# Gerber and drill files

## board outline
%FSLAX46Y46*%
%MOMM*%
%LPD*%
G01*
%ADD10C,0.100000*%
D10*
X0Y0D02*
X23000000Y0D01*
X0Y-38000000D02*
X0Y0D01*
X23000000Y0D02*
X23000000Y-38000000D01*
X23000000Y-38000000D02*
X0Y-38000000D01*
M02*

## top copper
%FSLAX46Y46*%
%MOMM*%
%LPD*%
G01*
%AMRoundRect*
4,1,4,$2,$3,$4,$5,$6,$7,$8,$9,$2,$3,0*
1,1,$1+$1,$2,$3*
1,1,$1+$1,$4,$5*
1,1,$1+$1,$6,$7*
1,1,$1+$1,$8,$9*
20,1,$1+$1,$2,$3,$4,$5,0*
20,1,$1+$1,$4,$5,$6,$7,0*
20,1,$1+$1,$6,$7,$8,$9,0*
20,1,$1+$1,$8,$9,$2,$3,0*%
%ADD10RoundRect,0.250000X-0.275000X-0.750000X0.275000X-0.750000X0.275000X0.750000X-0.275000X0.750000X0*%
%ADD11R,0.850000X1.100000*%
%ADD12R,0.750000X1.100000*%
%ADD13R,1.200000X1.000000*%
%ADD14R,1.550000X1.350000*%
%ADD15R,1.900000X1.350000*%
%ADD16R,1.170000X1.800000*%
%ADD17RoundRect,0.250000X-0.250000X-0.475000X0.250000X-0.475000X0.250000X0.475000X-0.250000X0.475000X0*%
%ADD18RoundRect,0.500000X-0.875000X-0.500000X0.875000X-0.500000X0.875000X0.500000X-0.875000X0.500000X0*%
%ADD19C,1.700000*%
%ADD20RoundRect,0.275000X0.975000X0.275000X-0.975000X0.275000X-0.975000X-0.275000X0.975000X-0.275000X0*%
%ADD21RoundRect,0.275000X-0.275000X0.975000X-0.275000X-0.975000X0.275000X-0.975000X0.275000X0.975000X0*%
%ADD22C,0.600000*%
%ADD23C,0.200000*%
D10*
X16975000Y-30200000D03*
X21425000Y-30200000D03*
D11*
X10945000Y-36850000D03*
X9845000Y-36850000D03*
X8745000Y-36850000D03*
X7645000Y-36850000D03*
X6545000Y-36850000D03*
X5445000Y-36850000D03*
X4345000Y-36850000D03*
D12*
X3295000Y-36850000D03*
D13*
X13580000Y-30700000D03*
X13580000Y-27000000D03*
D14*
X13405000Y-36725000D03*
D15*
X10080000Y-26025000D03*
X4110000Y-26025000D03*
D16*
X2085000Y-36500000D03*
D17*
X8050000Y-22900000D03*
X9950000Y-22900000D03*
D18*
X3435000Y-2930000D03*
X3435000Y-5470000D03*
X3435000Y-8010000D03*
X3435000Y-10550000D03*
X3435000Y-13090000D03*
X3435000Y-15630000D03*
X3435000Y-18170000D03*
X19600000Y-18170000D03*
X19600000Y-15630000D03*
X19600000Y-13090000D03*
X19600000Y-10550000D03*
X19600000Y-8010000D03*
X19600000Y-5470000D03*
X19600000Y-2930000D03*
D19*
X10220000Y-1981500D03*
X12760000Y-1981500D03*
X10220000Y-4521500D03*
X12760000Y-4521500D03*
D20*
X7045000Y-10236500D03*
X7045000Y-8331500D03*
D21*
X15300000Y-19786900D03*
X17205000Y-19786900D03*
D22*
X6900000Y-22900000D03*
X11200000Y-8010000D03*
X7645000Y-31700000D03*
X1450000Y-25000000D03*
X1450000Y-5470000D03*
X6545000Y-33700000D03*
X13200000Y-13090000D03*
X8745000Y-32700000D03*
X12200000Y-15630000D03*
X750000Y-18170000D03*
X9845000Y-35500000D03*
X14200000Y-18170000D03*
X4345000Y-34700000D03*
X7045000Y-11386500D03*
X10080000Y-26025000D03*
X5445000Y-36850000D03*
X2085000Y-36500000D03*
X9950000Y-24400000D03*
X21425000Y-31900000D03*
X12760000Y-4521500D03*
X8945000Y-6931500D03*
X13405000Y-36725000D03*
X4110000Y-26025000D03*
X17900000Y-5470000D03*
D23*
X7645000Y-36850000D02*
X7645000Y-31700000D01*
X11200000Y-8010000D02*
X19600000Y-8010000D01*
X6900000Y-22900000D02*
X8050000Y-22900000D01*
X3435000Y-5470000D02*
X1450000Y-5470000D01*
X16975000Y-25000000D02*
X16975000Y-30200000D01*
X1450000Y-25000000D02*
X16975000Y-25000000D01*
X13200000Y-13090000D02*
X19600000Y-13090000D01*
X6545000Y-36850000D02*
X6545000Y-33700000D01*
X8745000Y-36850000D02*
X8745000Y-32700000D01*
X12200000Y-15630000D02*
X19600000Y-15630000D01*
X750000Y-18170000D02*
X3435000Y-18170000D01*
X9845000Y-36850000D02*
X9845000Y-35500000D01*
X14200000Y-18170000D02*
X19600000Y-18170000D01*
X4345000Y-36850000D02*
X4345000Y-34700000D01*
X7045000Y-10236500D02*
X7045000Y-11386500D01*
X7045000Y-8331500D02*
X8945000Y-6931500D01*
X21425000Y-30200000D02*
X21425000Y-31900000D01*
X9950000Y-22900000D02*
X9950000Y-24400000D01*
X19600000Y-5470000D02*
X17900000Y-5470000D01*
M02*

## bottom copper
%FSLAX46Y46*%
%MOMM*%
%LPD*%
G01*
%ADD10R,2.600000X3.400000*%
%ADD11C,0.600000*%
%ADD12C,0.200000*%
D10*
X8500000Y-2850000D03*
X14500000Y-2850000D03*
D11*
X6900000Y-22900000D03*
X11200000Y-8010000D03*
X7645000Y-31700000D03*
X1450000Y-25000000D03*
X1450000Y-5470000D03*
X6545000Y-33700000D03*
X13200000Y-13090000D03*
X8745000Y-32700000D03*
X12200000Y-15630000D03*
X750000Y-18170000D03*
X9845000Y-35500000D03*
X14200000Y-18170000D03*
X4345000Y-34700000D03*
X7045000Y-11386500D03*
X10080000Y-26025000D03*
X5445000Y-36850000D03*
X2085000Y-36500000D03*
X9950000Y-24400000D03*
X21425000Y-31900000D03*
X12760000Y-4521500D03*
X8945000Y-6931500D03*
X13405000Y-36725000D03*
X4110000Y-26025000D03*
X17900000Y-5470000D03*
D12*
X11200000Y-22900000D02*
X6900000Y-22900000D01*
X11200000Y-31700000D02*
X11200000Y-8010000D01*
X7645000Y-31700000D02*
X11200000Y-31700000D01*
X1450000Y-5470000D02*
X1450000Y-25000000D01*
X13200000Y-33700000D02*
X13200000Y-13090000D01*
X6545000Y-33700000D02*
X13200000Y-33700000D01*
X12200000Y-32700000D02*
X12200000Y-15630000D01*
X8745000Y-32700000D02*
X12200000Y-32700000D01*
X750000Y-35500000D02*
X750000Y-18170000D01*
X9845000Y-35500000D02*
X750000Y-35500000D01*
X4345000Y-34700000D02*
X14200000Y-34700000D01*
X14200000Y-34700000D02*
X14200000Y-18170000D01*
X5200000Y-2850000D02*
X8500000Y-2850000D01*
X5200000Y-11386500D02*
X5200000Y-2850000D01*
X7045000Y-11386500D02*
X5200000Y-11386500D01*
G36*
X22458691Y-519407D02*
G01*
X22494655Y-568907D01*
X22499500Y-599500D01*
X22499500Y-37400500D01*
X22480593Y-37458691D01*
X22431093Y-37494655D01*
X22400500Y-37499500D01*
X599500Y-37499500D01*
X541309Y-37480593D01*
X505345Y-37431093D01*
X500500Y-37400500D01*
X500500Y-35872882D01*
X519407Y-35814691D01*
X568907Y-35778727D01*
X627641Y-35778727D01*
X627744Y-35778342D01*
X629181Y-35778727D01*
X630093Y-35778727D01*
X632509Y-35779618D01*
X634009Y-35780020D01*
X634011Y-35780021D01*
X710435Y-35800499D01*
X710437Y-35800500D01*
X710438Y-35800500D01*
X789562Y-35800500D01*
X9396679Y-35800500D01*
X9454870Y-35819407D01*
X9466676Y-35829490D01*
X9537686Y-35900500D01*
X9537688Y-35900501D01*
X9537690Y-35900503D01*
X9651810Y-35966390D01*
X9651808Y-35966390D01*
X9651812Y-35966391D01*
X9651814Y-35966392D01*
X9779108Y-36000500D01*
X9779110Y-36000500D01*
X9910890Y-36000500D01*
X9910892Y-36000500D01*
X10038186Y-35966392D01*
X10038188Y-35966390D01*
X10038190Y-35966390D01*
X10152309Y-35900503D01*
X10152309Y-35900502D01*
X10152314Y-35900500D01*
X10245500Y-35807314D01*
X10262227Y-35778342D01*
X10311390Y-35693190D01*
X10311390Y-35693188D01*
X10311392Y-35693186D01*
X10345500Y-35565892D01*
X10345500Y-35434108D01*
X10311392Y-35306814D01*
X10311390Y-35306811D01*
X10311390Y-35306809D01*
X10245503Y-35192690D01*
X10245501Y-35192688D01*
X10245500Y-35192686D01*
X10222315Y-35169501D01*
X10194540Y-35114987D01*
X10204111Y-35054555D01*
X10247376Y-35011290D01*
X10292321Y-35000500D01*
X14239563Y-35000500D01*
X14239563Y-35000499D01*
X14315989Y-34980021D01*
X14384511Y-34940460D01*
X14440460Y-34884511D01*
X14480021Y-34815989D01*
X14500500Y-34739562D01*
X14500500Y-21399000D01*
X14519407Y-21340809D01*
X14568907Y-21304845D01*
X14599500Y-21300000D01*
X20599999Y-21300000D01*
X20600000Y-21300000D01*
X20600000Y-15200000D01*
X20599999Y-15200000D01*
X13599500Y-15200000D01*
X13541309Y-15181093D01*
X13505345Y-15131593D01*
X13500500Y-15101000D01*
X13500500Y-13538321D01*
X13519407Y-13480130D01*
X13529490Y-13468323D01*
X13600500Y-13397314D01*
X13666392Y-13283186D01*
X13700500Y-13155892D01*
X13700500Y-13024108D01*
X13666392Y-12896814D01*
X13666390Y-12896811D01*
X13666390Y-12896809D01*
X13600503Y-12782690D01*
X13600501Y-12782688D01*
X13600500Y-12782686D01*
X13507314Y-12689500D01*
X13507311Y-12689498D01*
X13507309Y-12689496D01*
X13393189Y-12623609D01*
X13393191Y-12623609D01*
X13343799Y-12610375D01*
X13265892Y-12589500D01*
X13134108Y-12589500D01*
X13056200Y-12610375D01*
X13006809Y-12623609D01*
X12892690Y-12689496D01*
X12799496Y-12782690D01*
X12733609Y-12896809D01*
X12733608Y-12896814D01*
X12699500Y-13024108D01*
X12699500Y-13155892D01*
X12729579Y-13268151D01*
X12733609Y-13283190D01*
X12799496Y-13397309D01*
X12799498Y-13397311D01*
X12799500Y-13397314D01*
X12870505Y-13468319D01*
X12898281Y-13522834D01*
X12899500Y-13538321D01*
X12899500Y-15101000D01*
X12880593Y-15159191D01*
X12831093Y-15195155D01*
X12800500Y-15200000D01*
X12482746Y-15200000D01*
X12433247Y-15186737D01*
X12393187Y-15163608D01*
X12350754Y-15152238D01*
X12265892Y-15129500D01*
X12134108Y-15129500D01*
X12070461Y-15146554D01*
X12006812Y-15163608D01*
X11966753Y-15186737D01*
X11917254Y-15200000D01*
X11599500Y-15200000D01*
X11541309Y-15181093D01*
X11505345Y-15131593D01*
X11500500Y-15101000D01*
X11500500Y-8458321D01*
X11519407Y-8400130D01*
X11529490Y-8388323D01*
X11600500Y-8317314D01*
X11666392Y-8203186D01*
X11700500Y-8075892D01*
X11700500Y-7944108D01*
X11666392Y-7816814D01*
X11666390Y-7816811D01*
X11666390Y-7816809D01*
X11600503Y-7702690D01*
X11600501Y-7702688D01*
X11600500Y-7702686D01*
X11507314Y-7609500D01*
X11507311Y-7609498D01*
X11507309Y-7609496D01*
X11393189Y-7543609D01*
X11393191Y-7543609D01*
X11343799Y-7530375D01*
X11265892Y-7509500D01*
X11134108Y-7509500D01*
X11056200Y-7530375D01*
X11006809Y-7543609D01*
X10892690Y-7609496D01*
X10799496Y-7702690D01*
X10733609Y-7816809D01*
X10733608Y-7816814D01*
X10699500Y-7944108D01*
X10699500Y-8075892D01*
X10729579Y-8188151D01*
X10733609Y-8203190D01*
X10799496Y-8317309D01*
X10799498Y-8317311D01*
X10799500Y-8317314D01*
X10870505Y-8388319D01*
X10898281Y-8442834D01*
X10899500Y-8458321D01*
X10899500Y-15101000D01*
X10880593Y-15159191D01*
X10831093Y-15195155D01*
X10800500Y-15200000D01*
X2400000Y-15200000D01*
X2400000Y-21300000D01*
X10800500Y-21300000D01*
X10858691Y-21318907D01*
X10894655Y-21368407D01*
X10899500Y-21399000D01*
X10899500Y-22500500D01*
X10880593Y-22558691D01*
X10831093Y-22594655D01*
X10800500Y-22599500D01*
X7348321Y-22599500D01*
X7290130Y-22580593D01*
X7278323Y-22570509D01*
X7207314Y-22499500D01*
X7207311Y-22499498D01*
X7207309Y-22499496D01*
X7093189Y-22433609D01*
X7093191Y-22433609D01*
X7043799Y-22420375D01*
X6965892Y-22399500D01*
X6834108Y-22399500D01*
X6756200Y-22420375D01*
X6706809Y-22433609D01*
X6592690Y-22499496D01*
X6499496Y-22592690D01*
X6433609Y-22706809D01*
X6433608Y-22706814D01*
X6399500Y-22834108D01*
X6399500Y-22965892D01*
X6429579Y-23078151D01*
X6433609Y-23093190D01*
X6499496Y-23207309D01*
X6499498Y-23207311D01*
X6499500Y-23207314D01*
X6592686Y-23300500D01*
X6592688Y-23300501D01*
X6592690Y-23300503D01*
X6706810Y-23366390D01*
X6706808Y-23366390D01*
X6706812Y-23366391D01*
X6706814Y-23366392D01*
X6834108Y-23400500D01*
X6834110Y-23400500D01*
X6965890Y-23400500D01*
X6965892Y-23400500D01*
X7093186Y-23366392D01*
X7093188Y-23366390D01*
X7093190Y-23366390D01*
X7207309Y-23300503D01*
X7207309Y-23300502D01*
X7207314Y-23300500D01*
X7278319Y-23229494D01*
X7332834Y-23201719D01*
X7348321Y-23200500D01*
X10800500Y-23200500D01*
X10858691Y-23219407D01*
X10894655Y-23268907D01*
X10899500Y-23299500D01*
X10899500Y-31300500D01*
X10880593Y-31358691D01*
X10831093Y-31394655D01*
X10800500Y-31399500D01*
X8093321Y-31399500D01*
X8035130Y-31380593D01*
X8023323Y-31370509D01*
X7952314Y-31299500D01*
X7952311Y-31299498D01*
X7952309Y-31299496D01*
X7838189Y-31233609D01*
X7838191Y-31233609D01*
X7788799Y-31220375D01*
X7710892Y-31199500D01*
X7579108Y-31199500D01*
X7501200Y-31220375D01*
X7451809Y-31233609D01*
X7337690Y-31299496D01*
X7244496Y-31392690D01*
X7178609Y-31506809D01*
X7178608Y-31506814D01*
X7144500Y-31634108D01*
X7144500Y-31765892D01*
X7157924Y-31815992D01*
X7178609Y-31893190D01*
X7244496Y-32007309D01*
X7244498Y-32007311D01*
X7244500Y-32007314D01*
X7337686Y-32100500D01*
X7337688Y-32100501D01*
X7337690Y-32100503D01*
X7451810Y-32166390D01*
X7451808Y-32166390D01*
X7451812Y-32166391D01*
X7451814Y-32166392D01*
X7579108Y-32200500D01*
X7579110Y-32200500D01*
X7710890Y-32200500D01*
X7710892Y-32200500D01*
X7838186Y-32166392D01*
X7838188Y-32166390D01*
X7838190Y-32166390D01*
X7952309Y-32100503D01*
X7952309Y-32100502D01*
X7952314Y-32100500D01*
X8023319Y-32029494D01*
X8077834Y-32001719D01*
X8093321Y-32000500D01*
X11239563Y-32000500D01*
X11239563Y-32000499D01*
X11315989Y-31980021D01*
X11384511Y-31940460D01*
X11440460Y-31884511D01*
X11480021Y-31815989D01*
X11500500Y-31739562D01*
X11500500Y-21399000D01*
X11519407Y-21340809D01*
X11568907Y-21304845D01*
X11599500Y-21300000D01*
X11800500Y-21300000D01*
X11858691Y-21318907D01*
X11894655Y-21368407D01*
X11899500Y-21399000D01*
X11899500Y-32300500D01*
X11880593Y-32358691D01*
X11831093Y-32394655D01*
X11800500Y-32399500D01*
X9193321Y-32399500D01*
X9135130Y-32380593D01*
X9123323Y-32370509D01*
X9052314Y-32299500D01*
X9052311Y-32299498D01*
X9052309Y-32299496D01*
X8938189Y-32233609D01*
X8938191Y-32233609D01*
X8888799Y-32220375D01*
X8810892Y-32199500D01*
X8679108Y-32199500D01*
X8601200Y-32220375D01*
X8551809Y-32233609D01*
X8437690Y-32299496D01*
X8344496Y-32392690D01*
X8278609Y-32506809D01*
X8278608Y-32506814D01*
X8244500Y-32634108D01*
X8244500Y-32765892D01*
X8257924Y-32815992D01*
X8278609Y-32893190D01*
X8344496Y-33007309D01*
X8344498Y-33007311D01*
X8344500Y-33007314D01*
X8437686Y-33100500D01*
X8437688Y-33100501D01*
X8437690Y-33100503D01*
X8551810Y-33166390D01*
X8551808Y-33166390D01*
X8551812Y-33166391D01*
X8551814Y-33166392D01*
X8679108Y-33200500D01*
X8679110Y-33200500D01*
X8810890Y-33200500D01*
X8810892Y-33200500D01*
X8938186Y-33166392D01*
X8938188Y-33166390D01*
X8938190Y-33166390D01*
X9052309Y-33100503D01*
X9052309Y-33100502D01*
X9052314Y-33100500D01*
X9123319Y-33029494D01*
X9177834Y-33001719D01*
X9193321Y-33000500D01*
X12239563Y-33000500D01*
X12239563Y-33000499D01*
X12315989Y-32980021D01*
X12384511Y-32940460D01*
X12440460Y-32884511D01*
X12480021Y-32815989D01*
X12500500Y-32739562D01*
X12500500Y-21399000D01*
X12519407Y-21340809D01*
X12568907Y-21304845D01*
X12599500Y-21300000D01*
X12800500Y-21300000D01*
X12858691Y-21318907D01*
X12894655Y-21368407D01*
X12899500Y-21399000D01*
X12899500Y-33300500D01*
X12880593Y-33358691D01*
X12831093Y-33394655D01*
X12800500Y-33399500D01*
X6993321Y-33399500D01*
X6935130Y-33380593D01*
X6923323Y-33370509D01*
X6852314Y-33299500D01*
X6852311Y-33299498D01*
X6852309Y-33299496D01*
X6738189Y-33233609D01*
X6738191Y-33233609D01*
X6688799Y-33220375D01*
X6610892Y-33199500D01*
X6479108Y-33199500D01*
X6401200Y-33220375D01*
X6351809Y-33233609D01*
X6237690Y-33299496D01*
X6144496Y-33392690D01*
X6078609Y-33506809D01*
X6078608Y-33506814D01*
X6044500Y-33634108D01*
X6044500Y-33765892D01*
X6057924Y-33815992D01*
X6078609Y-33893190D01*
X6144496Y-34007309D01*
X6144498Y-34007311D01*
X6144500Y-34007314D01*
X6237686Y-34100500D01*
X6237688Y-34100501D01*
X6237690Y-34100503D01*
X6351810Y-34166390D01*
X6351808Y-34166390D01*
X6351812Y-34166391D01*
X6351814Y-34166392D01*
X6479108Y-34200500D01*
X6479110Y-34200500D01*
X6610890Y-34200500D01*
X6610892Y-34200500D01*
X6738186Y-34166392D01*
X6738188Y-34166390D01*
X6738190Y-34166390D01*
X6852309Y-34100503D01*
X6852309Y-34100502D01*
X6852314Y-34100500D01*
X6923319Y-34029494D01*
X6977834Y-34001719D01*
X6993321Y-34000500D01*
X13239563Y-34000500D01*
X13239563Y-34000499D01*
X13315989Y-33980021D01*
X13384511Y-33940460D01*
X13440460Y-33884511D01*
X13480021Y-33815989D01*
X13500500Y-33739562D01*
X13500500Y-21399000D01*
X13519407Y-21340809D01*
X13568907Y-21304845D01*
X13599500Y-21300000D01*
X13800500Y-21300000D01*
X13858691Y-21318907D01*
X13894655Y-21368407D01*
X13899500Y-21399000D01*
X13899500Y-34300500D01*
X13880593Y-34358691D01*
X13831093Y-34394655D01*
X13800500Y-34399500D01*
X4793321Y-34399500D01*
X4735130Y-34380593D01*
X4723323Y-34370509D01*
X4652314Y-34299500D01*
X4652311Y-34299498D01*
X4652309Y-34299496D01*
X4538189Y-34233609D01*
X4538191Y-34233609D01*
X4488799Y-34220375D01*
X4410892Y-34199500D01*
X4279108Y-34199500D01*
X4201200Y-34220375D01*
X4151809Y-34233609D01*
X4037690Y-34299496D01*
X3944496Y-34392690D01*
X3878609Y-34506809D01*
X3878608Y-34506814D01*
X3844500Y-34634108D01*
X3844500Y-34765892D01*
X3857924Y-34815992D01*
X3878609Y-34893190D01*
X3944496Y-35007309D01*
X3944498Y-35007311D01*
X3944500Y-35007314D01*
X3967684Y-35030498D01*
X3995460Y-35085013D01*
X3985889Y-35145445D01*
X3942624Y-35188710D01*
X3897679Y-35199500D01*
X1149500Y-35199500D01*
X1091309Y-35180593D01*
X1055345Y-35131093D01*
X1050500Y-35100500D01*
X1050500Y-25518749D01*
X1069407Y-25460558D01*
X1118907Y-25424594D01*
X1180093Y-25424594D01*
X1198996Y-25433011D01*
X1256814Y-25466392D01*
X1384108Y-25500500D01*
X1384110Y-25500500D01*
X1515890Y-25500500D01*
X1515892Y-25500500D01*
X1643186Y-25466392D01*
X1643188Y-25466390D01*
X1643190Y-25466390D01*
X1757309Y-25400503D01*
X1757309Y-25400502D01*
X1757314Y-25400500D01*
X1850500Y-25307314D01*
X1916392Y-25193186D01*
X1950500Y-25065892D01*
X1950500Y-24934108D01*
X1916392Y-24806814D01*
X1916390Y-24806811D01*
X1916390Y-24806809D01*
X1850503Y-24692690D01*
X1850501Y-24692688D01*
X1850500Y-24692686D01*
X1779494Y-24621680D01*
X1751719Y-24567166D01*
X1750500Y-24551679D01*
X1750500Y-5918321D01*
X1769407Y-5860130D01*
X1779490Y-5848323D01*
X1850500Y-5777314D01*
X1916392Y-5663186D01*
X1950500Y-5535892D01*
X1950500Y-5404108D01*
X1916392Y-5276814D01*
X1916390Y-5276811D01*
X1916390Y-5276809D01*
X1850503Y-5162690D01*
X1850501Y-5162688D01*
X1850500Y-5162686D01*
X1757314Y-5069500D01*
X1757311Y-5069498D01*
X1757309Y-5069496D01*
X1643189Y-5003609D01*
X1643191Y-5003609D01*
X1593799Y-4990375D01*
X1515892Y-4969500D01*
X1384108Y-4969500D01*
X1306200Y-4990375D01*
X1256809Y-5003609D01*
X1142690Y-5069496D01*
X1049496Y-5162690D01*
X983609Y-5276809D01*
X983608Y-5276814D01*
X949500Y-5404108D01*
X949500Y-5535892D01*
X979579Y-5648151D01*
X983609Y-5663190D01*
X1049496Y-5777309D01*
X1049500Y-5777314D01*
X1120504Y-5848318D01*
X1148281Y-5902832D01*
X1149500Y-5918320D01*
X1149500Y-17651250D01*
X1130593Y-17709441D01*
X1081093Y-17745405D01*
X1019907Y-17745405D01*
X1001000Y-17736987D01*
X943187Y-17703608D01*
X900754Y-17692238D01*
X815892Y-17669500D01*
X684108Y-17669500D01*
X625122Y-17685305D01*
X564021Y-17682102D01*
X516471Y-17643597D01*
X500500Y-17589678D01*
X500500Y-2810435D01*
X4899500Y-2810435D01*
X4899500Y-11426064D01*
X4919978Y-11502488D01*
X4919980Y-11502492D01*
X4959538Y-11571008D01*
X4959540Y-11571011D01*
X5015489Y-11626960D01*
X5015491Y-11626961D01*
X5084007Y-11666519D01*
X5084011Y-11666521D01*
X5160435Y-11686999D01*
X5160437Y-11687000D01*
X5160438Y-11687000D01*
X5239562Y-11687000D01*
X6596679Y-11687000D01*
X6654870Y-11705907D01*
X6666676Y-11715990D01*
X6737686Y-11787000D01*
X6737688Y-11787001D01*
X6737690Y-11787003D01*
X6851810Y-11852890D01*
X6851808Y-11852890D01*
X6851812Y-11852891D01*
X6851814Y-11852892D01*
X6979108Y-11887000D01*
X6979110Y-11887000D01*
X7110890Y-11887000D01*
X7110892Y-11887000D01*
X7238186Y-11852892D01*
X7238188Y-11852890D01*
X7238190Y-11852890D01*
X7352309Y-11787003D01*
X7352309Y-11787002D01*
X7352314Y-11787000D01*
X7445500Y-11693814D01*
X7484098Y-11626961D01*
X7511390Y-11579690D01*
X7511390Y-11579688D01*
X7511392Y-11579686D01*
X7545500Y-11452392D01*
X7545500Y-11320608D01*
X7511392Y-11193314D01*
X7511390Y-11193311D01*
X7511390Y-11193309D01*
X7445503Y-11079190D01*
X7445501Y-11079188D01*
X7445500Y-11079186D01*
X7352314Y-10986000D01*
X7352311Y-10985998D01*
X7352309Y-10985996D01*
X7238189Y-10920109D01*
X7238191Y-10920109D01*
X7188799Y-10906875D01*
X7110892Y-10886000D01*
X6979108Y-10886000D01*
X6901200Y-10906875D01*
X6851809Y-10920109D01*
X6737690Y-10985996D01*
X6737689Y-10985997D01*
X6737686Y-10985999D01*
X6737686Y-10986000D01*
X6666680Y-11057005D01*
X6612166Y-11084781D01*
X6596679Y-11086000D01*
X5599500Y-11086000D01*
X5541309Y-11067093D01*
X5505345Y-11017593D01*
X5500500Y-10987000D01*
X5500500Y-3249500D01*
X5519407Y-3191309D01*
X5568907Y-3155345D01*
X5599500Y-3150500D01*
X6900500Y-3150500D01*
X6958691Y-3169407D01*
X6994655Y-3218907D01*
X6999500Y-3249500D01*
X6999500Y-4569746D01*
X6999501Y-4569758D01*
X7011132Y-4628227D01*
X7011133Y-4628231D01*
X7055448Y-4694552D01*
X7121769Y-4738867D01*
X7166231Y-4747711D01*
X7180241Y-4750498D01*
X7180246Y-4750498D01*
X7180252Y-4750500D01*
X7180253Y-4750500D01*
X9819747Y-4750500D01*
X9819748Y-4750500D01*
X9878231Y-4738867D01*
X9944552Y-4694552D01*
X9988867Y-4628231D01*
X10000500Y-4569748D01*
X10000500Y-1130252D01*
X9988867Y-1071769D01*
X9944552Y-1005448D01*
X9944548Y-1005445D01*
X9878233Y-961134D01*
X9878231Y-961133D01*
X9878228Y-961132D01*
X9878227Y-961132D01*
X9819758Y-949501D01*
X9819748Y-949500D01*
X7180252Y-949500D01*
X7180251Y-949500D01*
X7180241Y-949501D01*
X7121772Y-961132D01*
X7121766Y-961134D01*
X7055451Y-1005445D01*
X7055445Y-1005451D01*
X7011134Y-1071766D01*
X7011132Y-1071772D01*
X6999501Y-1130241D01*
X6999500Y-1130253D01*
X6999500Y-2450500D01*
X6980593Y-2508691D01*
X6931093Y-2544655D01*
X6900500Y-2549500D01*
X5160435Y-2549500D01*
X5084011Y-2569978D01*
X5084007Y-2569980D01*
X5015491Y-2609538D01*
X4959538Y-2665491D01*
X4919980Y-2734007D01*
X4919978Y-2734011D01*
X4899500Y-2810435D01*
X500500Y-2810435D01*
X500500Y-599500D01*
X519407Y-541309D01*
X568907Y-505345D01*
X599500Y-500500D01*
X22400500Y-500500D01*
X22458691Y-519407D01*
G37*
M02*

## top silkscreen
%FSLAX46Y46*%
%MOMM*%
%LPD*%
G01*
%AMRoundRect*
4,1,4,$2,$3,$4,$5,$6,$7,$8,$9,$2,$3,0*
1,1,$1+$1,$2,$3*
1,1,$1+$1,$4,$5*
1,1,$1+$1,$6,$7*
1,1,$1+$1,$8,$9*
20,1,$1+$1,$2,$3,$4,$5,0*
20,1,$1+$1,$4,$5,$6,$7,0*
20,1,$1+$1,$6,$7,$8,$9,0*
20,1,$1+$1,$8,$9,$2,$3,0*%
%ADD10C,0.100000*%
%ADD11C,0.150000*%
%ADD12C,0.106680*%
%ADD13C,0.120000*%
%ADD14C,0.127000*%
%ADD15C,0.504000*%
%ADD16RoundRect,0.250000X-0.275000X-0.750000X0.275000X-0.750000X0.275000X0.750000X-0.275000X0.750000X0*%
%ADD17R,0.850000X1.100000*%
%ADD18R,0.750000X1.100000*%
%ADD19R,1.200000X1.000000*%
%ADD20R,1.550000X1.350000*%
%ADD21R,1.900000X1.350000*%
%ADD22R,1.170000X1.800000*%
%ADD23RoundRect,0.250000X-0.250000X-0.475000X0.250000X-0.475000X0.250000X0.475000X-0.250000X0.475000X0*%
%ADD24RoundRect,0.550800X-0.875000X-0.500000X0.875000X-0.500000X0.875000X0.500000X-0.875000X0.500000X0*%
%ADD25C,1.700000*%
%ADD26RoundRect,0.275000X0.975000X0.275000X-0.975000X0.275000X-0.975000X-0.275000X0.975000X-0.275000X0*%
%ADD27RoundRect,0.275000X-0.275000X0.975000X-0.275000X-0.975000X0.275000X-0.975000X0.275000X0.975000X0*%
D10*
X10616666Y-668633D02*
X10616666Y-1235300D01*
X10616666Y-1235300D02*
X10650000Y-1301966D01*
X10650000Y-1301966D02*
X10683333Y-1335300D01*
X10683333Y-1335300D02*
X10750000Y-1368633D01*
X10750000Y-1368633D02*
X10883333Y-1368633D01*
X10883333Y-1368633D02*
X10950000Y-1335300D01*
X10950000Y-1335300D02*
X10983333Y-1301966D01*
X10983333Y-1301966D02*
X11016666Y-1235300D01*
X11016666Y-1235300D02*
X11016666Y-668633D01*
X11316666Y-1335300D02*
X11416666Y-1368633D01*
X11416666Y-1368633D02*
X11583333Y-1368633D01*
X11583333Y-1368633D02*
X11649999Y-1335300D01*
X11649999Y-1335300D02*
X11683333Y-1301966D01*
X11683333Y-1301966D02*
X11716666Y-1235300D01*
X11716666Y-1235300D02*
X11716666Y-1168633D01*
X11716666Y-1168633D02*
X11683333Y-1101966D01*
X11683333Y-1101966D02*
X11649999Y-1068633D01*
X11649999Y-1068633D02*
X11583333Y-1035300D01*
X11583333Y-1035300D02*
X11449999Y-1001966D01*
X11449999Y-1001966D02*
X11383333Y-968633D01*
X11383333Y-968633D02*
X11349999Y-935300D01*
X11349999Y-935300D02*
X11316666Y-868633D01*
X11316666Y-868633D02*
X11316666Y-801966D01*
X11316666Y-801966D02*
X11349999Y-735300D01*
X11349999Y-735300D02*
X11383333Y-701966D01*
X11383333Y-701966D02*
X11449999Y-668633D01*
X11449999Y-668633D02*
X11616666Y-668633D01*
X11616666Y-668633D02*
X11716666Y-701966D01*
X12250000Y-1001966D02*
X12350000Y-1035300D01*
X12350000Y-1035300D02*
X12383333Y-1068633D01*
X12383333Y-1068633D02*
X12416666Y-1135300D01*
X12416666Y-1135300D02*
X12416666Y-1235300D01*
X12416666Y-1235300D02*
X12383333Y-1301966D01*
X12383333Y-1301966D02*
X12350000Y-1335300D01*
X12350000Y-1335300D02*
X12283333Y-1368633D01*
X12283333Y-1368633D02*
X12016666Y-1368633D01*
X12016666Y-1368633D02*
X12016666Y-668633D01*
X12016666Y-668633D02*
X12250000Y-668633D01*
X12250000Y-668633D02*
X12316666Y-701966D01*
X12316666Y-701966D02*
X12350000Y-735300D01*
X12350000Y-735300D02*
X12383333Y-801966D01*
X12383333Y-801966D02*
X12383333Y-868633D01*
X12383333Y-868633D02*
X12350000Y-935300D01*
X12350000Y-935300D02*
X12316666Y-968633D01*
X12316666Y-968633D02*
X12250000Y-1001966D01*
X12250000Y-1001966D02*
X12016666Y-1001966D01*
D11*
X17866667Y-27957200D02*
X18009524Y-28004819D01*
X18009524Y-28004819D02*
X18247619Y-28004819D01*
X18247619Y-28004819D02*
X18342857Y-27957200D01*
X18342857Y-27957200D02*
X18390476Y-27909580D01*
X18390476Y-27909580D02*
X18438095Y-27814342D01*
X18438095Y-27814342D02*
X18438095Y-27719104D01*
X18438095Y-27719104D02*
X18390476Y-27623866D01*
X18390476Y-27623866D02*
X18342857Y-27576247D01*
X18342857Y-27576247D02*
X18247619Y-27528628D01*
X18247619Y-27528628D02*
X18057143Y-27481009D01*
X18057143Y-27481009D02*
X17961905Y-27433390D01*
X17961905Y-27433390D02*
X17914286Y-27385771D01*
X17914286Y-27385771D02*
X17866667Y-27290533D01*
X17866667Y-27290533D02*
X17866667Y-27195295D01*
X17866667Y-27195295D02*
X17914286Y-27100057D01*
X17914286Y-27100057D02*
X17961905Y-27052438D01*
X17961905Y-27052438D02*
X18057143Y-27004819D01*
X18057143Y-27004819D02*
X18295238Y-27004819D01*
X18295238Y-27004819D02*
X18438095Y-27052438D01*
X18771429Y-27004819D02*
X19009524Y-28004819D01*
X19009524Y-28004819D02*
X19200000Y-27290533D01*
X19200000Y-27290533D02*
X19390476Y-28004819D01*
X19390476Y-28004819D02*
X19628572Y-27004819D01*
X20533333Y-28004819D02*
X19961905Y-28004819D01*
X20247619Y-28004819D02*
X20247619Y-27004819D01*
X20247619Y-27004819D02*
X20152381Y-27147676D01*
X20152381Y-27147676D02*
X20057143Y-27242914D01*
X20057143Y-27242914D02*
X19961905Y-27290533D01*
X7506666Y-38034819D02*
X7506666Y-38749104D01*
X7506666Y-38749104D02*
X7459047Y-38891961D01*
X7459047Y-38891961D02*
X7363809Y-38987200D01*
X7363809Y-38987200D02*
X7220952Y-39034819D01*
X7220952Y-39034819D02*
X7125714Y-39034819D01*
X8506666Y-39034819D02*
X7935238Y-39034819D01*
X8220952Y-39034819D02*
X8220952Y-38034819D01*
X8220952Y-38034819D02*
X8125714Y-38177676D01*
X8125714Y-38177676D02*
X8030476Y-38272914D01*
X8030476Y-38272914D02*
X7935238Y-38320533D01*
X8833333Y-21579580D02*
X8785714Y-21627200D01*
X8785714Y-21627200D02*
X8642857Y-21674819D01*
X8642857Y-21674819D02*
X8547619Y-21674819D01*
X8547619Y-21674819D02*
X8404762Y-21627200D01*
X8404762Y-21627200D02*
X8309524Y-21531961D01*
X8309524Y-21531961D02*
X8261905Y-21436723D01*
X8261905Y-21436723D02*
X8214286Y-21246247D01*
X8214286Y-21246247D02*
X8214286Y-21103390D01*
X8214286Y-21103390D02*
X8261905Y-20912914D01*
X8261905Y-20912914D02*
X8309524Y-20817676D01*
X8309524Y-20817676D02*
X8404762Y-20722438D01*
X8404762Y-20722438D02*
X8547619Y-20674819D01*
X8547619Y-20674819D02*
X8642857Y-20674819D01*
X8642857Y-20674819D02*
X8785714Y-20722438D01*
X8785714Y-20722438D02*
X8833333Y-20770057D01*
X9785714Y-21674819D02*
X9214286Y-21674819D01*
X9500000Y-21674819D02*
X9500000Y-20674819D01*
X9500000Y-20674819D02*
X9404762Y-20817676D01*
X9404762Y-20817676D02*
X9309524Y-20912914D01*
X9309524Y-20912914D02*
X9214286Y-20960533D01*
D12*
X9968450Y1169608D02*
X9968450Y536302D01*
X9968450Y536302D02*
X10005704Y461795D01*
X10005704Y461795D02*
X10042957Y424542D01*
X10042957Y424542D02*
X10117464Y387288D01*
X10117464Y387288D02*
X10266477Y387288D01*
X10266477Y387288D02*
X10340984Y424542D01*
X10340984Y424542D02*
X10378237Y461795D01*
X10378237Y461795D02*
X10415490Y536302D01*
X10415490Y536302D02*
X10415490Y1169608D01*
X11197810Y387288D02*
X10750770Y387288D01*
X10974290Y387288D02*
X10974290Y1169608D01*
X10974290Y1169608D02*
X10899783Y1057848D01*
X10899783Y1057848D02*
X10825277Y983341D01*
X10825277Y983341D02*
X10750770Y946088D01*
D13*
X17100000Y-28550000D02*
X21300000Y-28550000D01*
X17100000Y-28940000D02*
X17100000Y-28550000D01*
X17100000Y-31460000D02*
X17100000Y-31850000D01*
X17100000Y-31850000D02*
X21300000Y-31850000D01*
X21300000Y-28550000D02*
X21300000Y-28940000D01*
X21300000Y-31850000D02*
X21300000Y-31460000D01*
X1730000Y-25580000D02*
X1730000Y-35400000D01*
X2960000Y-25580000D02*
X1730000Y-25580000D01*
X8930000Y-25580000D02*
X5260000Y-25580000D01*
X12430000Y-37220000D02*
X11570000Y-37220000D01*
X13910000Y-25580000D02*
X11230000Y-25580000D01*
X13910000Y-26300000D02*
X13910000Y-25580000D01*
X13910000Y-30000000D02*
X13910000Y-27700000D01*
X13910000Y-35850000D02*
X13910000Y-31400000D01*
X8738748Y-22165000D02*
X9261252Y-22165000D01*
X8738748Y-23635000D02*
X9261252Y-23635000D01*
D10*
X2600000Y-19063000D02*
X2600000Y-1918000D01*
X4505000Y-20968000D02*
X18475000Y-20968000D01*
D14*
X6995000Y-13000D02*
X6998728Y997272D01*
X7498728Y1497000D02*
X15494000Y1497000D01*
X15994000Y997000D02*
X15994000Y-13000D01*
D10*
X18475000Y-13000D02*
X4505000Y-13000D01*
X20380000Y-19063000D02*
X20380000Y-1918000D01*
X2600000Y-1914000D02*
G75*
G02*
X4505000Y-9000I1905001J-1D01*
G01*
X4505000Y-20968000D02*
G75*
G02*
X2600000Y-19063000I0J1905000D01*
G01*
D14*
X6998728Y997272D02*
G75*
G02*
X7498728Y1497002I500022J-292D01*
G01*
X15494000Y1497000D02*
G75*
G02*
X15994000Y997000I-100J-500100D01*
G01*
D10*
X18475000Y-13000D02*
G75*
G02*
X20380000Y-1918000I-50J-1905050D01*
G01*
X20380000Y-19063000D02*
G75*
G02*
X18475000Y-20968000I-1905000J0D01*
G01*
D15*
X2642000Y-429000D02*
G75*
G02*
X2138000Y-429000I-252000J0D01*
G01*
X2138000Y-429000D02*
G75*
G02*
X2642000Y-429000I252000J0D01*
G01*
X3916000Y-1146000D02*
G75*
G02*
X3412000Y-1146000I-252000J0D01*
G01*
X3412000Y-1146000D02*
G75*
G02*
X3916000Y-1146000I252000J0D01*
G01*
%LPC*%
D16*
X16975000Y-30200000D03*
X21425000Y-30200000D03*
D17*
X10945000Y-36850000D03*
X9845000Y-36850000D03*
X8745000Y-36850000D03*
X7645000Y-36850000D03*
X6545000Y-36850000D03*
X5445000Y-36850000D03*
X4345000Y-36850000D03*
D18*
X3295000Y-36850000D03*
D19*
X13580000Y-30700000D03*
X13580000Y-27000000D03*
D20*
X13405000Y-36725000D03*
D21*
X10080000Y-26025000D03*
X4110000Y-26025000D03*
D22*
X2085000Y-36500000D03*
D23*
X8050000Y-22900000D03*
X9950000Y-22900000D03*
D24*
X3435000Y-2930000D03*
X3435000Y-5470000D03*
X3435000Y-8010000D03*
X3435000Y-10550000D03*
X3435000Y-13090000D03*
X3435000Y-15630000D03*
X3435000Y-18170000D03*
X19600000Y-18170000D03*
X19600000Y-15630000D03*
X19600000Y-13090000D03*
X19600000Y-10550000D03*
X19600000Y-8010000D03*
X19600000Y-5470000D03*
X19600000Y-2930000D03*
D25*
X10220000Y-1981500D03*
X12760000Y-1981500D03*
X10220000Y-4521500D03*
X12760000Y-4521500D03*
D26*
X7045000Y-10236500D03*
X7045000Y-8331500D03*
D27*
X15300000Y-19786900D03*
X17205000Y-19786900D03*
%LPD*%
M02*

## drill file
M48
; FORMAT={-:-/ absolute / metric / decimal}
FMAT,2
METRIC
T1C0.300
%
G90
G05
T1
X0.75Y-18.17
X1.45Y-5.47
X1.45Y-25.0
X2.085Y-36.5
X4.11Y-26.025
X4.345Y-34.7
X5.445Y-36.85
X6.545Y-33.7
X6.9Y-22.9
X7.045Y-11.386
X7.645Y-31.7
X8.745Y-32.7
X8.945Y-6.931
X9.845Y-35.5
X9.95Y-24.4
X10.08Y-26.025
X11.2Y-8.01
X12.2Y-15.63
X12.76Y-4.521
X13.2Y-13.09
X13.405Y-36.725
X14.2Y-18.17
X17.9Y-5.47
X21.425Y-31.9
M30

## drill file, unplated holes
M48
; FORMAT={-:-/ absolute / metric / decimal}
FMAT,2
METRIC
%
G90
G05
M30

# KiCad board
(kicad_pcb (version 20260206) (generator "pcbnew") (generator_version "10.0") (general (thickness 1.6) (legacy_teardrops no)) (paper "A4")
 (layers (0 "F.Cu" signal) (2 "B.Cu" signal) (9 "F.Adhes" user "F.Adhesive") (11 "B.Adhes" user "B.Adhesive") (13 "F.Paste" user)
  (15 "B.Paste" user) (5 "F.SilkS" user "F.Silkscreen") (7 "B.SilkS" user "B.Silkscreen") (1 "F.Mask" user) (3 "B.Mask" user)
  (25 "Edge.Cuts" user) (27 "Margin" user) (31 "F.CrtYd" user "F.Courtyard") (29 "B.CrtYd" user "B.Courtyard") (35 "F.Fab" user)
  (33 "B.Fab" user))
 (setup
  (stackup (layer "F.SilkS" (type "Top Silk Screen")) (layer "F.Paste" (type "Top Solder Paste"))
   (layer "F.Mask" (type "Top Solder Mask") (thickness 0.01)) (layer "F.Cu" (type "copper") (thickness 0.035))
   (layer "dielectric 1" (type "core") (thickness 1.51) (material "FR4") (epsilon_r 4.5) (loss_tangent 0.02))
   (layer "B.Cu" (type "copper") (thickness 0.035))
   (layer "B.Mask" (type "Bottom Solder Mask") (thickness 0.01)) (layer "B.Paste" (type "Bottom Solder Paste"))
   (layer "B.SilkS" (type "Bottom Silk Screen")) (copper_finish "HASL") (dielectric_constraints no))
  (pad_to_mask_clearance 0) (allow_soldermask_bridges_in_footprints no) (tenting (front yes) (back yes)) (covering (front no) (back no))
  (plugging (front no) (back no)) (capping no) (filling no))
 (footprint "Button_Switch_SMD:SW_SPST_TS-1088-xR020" (layer "F.Cu") (at 19.2 30.2)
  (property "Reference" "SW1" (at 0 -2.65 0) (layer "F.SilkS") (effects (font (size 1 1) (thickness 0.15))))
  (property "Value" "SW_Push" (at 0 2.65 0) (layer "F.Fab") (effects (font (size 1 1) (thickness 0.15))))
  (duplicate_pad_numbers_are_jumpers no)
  (fp_line (start -2.1 -1.65) (end 2.1 -1.65) (stroke (width 0.12) (type solid)) (layer "F.SilkS"))
  (fp_line (start -2.1 -1.26) (end -2.1 -1.65) (stroke (width 0.12) (type solid)) (layer "F.SilkS"))
  (fp_line (start -2.1 1.26) (end -2.1 1.65) (stroke (width 0.12) (type solid)) (layer "F.SilkS"))
  (fp_line (start -2.1 1.65) (end 2.1 1.65) (stroke (width 0.12) (type solid)) (layer "F.SilkS"))
  (fp_line (start 2.1 -1.65) (end 2.1 -1.26) (stroke (width 0.12) (type solid)) (layer "F.SilkS"))
  (fp_line (start 2.1 1.65) (end 2.1 1.26) (stroke (width 0.12) (type solid)) (layer "F.SilkS"))
  (pad "1" smd roundrect (at -2.225 0) (size 1.05 2) (layers "F.Cu" "F.Mask" "F.Paste") (roundrect_rratio 0.2380952381) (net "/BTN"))
  (pad "2" smd roundrect (at 2.225 0) (size 1.05 2) (layers "F.Cu" "F.Mask" "F.Paste") (roundrect_rratio 0.2380952381) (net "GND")))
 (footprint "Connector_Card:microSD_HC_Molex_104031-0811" (layer "F.Cu") (at 7.84 31.4 180)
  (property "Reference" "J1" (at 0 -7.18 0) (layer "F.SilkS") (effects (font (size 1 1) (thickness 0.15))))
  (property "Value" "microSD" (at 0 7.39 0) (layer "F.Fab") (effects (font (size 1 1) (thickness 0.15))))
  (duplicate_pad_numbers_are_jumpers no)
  (fp_line (start 6.11 5.82) (end 6.11 -4) (stroke (width 0.12) (type solid)) (layer "F.SilkS"))
  (fp_line (start 4.88 5.82) (end 6.11 5.82) (stroke (width 0.12) (type solid)) (layer "F.SilkS"))
  (fp_line (start -1.09 5.82) (end 2.58 5.82) (stroke (width 0.12) (type solid)) (layer "F.SilkS"))
  (fp_line (start -4.59 -5.82) (end -3.73 -5.82) (stroke (width 0.12) (type solid)) (layer "F.SilkS"))
  (fp_line (start -6.07 5.82) (end -3.39 5.82) (stroke (width 0.12) (type solid)) (layer "F.SilkS"))
  (fp_line (start -6.07 5.1) (end -6.07 5.82) (stroke (width 0.12) (type solid)) (layer "F.SilkS"))
  (fp_line (start -6.07 1.4) (end -6.07 3.7) (stroke (width 0.12) (type solid)) (layer "F.SilkS"))
  (fp_line (start -6.07 -4.45) (end -6.07 0) (stroke (width 0.12) (type solid)) (layer "F.SilkS"))
  (pad "1" smd rect (at -3.105 -5.45) (size 0.85 1.1) (layers "F.Cu" "F.Mask" "F.Paste"))
  (pad "2" smd rect (at -2.005 -5.45) (size 0.85 1.1) (layers "F.Cu" "F.Mask" "F.Paste") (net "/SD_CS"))
  (pad "3" smd rect (at -0.905 -5.45) (size 0.85 1.1) (layers "F.Cu" "F.Mask" "F.Paste") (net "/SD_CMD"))
  (pad "4" smd rect (at 0.195 -5.45) (size 0.85 1.1) (layers "F.Cu" "F.Mask" "F.Paste") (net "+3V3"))
  (pad "5" smd rect (at 1.295 -5.45) (size 0.85 1.1) (layers "F.Cu" "F.Mask" "F.Paste") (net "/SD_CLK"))
  (pad "6" smd rect (at 2.395 -5.45) (size 0.85 1.1) (layers "F.Cu" "F.Mask" "F.Paste") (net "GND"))
  (pad "7" smd rect (at 3.495 -5.45) (size 0.85 1.1) (layers "F.Cu" "F.Mask" "F.Paste") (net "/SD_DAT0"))
  (pad "8" smd rect (at 4.545 -5.45) (size 0.75 1.1) (layers "F.Cu" "F.Mask" "F.Paste"))
  (pad "9" smd rect (at -5.74 0.7) (size 1.2 1) (layers "F.Cu" "F.Mask" "F.Paste"))
  (pad "10" smd rect (at -5.74 4.4) (size 1.2 1) (layers "F.Cu" "F.Mask" "F.Paste"))
  (pad "SH" smd rect (at -5.565 -5.325) (size 1.55 1.35) (layers "F.Cu" "F.Mask" "F.Paste") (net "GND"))
  (pad "SH" smd rect (at -2.24 5.375) (size 1.9 1.35) (layers "F.Cu" "F.Mask" "F.Paste") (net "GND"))
  (pad "SH" smd rect (at 3.73 5.375) (size 1.9 1.35) (layers "F.Cu" "F.Mask" "F.Paste") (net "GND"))
  (pad "SH" smd rect (at 5.755 -5.1) (size 1.17 1.8) (layers "F.Cu" "F.Mask" "F.Paste") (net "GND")))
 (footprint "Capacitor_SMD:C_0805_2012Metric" (layer "F.Cu") (at 9 22.9)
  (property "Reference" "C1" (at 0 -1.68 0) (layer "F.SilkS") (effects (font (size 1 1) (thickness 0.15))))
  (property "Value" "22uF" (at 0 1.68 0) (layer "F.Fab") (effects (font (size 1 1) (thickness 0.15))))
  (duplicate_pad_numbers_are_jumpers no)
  (fp_line (start -0.261252 -0.735) (end 0.261252 -0.735) (stroke (width 0.12) (type solid)) (layer "F.SilkS"))
  (fp_line (start -0.261252 0.735) (end 0.261252 0.735) (stroke (width 0.12) (type solid)) (layer "F.SilkS"))
  (pad "1" smd roundrect (at -0.95 0) (size 1 1.45) (layers "F.Cu" "F.Mask" "F.Paste") (roundrect_rratio 0.25) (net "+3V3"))
  (pad "2" smd roundrect (at 0.95 0) (size 1 1.45) (layers "F.Cu" "F.Mask" "F.Paste") (roundrect_rratio 0.25) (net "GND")))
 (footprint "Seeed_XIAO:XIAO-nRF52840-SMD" (layer "F.Cu") (at 2.6 21.05)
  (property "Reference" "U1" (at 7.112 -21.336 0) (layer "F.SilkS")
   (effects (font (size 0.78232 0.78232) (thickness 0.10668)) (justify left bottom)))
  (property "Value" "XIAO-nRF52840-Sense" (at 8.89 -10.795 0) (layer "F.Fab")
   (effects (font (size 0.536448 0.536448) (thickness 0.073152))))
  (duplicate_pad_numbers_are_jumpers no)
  (fp_line (start 0 -1.987) (end 0 -19.132) (stroke (width 0.1) (type solid)) (layer "F.SilkS"))
  (fp_line (start 1.905 -0.082) (end 15.875 -0.082) (stroke (width 0.1) (type solid)) (layer "F.SilkS"))
  (fp_line (start 4.395 -21.037) (end 4.398728 -22.047272) (stroke (width 0.127) (type solid)) (layer "F.SilkS"))
  (fp_line (start 4.898728 -22.547) (end 12.894 -22.547) (stroke (width 0.127) (type solid)) (layer "F.SilkS"))
  (fp_line (start 13.394 -22.047) (end 13.394 -21.037) (stroke (width 0.127) (type solid)) (layer "F.SilkS"))
  (fp_line (start 15.875 -21.037) (end 1.905 -21.037) (stroke (width 0.1) (type solid)) (layer "F.SilkS"))
  (fp_line (start 17.78 -1.987) (end 17.78 -19.132) (stroke (width 0.1) (type solid)) (layer "F.SilkS"))
  (fp_arc (start 0 -19.136) (mid 0.557962 -20.483038) (end 1.905 -21.041) (stroke (width 0.1) (type solid)) (layer "F.SilkS"))
  (fp_arc (start 1.905 -0.082) (mid 0.557962 -0.639962) (end 0 -1.987) (stroke (width 0.1) (type solid)) (layer "F.SilkS"))
  (fp_arc (start 4.398728 -22.047272) (mid 4.545276 -22.400644) (end 4.898728 -22.547) (stroke (width 0.127) (type default))
   (layer "F.SilkS"))
  (fp_arc (start 12.894 -22.547) (mid 13.247531 -22.400546) (end 13.394 -22.047) (stroke (width 0.127) (type default)) (layer "F.SilkS"))
  (fp_arc (start 15.875 -21.037) (mid 17.222016 -20.479031) (end 17.78 -19.132) (stroke (width 0.1) (type solid)) (layer "F.SilkS"))
  (fp_arc (start 17.78 -1.987) (mid 17.222038 -0.639961) (end 15.875 -0.082) (stroke (width 0.1) (type solid)) (layer "F.SilkS"))
  (fp_circle (center -0.21 -20.621) (end -0.21 -20.875) (stroke (width 0.5) (type solid)) (fill yes) (layer "F.SilkS"))
  (fp_circle (center 1.064 -19.904) (end 1.064 -20.158) (stroke (width 0.5) (type solid)) (fill yes) (layer "F.SilkS"))
  (pad "1" smd roundrect (at 0.835 -18.12) (size 2.75 2) (layers "F.Cu" "F.Mask" "F.Paste") (roundrect_rratio 0.25)
   (solder_mask_margin 0.0508) (thermal_bridge_angle 45))
  (pad "2" smd roundrect (at 0.835 -15.58) (size 2.75 2) (layers "F.Cu" "F.Mask" "F.Paste") (roundrect_rratio 0.25) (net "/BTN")
   (solder_mask_margin 0.0508) (thermal_bridge_angle 45))
  (pad "3" smd roundrect (at 0.835 -13.04) (size 2.75 2) (layers "F.Cu" "F.Mask" "F.Paste") (roundrect_rratio 0.25)
   (solder_mask_margin 0.0508) (thermal_bridge_angle 45))
  (pad "4" smd roundrect (at 0.835 -10.5) (size 2.75 2) (layers "F.Cu" "F.Mask" "F.Paste") (roundrect_rratio 0.25)
   (solder_mask_margin 0.0508) (thermal_bridge_angle 45))
  (pad "5" smd roundrect (at 0.835 -7.96) (size 2.75 2) (layers "F.Cu" "F.Mask" "F.Paste") (roundrect_rratio 0.25)
   (solder_mask_margin 0.0508) (thermal_bridge_angle 45))
  (pad "6" smd roundrect (at 0.835 -5.42) (size 2.75 2) (layers "F.Cu" "F.Mask" "F.Paste") (roundrect_rratio 0.25)
   (solder_mask_margin 0.0508) (thermal_bridge_angle 45))
  (pad "7" smd roundrect (at 0.835 -2.88) (size 2.75 2) (layers "F.Cu" "F.Mask" "F.Paste") (roundrect_rratio 0.25) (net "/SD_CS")
   (solder_mask_margin 0.0508) (thermal_bridge_angle 45))
  (pad "8" smd roundrect (at 17 -2.88) (size 2.75 2) (layers "F.Cu" "F.Mask" "F.Paste") (roundrect_rratio 0.25) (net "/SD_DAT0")
   (solder_mask_margin 0.0508) (thermal_bridge_angle 45))
  (pad "9" smd roundrect (at 17 -5.42) (size 2.75 2) (layers "F.Cu" "F.Mask" "F.Paste") (roundrect_rratio 0.25) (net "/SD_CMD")
   (solder_mask_margin 0.0508) (thermal_bridge_angle 45))
  (pad "10" smd roundrect (at 17 -7.96) (size 2.75 2) (layers "F.Cu" "F.Mask" "F.Paste") (roundrect_rratio 0.25) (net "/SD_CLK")
   (solder_mask_margin 0.0508) (thermal_bridge_angle 45))
  (pad "11" smd roundrect (at 17 -10.5) (size 2.75 2) (layers "F.Cu" "F.Mask" "F.Paste") (roundrect_rratio 0.25) (solder_mask_margin 0.0508)
   (thermal_bridge_angle 45))
  (pad "12" smd roundrect (at 17 -13.04) (size 2.75 2) (layers "F.Cu" "F.Mask" "F.Paste") (roundrect_rratio 0.25) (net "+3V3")
   (solder_mask_margin 0.0508) (thermal_bridge_angle 45))
  (pad "13" smd roundrect (at 17 -15.58) (size 2.75 2) (layers "F.Cu" "F.Mask" "F.Paste") (roundrect_rratio 0.25) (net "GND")
   (solder_mask_margin 0.0508) (thermal_bridge_angle 45))
  (pad "14" smd roundrect (at 17 -18.12) (size 2.75 2) (layers "F.Cu" "F.Mask" "F.Paste") (roundrect_rratio 0.25)
   (solder_mask_margin 0.0508) (thermal_bridge_angle 45))
  (pad "15" smd circle (at 7.62 -19.0685) (size 1.7 1.7) (layers "F.Cu" "F.Mask" "F.Paste"))
  (pad "16" smd circle (at 10.16 -19.0685) (size 1.7 1.7) (layers "F.Cu" "F.Mask" "F.Paste"))
  (pad "17" smd circle (at 7.62 -16.5285) (size 1.7 1.7) (layers "F.Cu" "F.Mask" "F.Paste"))
  (pad "18" smd circle (at 10.16 -16.5285) (size 1.7 1.7) (layers "F.Cu" "F.Mask" "F.Paste") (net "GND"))
  (pad "19" smd roundrect (at 4.445 -10.8135 180) (size 2.5 1.1) (layers "F.Cu" "F.Mask" "F.Paste") (roundrect_rratio 0.25) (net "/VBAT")
   (thermal_bridge_angle 45))
  (pad "20" smd roundrect (at 4.445 -12.7185 180) (size 2.5 1.1) (layers "F.Cu" "F.Mask" "F.Paste") (roundrect_rratio 0.25) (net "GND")
   (thermal_bridge_angle 45))
  (pad "21" smd roundrect (at 12.7 -1.2631 270) (size 2.5 1.1) (layers "F.Cu" "F.Mask" "F.Paste") (roundrect_rratio 0.25)
   (thermal_bridge_angle 45))
  (pad "22" smd roundrect (at 14.605 -1.2631 270) (size 2.5 1.1) (layers "F.Cu" "F.Mask" "F.Paste") (roundrect_rratio 0.25)
   (thermal_bridge_angle 45)))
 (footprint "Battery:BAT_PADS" (layer "F.Cu") (at 11.5 2.85)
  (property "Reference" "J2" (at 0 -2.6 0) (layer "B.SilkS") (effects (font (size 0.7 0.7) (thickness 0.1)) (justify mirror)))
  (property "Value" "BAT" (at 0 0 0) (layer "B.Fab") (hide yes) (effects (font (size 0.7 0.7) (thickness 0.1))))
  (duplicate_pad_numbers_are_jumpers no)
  (pad "1" smd rect (at -3 0) (size 2.6 3.4) (layers "B.Cu" "B.Mask" "B.Paste") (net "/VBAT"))
  (pad "2" smd rect (at 3 0) (size 2.6 3.4) (layers "B.Cu" "B.Mask" "B.Paste") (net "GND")))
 (gr_line (start 0 0) (end 23 0) (stroke (width 0.1) (type default)) (layer "Edge.Cuts"))
 (gr_line (start 0 38) (end 0 0) (stroke (width 0.1) (type default)) (layer "Edge.Cuts"))
 (gr_line (start 23 0) (end 23 38) (stroke (width 0.1) (type default)) (layer "Edge.Cuts"))
 (gr_line (start 23 38) (end 0 38) (stroke (width 0.1) (type default)) (layer "Edge.Cuts"))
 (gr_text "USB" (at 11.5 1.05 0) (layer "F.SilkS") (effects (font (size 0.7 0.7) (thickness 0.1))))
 (segment (start 7.645 36.85) (end 7.645 31.7) (width 0.2) (layer "F.Cu") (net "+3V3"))
 (segment (start 11.2 8.01) (end 19.6 8.01) (width 0.2) (layer "F.Cu") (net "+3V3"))
 (segment (start 6.9 22.9) (end 8.05 22.9) (width 0.2) (layer "F.Cu") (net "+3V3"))
 (via (at 6.9 22.9) (size 0.6) (drill 0.3) (layers "F.Cu" "B.Cu") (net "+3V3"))
 (via (at 11.2 8.01) (size 0.6) (drill 0.3) (layers "F.Cu" "B.Cu") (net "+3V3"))
 (via (at 7.645 31.7) (size 0.6) (drill 0.3) (layers "F.Cu" "B.Cu") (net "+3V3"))
 (segment (start 11.2 22.9) (end 6.9 22.9) (width 0.2) (layer "B.Cu") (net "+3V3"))
 (segment (start 11.2 31.7) (end 11.2 8.01) (width 0.2) (layer "B.Cu") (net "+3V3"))
 (segment (start 7.645 31.7) (end 11.2 31.7) (width 0.2) (layer "B.Cu") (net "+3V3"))
 (segment (start 3.435 5.47) (end 1.45 5.47) (width 0.2) (layer "F.Cu") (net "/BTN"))
 (segment (start 16.975 25) (end 16.975 30.2) (width 0.2) (layer "F.Cu") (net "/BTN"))
 (segment (start 1.45 25) (end 16.975 25) (width 0.2) (layer "F.Cu") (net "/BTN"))
 (via (at 1.45 25) (size 0.6) (drill 0.3) (layers "F.Cu" "B.Cu") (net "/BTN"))
 (via (at 1.45 5.47) (size 0.6) (drill 0.3) (layers "F.Cu" "B.Cu") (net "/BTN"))
 (segment (start 1.45 5.47) (end 1.45 25) (width 0.2) (layer "B.Cu") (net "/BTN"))
 (segment (start 13.2 13.09) (end 19.6 13.09) (width 0.2) (layer "F.Cu") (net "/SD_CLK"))
 (segment (start 6.545 36.85) (end 6.545 33.7) (width 0.2) (layer "F.Cu") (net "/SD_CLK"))
 (via (at 6.545 33.7) (size 0.6) (drill 0.3) (layers "F.Cu" "B.Cu") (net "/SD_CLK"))
 (via (at 13.2 13.09) (size 0.6) (drill 0.3) (layers "F.Cu" "B.Cu") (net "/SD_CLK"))
 (segment (start 13.2 33.7) (end 13.2 13.09) (width 0.2) (layer "B.Cu") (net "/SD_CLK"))
 (segment (start 6.545 33.7) (end 13.2 33.7) (width 0.2) (layer "B.Cu") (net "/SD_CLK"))
 (segment (start 8.745 36.85) (end 8.745 32.7) (width 0.2) (layer "F.Cu") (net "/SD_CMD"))
 (segment (start 12.2 15.63) (end 19.6 15.63) (width 0.2) (layer "F.Cu") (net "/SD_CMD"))
 (via (at 8.745 32.7) (size 0.6) (drill 0.3) (layers "F.Cu" "B.Cu") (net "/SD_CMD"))
 (via (at 12.2 15.63) (size 0.6) (drill 0.3) (layers "F.Cu" "B.Cu") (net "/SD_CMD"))
 (segment (start 12.2 32.7) (end 12.2 15.63) (width 0.2) (layer "B.Cu") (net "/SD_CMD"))
 (segment (start 8.745 32.7) (end 12.2 32.7) (width 0.2) (layer "B.Cu") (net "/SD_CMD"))
 (segment (start 0.75 18.17) (end 3.435 18.17) (width 0.2) (layer "F.Cu") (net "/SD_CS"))
 (segment (start 9.845 36.85) (end 9.845 35.5) (width 0.2) (layer "F.Cu") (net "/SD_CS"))
 (via (at 0.75 18.17) (size 0.6) (drill 0.3) (layers "F.Cu" "B.Cu") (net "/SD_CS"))
 (via (at 9.845 35.5) (size 0.6) (drill 0.3) (layers "F.Cu" "B.Cu") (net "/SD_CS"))
 (segment (start 0.75 35.5) (end 0.75 18.17) (width 0.2) (layer "B.Cu") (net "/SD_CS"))
 (segment (start 9.845 35.5) (end 0.75 35.5) (width 0.2) (layer "B.Cu") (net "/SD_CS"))
 (segment (start 14.2 18.17) (end 19.6 18.17) (width 0.2) (layer "F.Cu") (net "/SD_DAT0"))
 (segment (start 4.345 36.85) (end 4.345 34.7) (width 0.2) (layer "F.Cu") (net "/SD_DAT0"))
 (via (at 14.2 18.17) (size 0.6) (drill 0.3) (layers "F.Cu" "B.Cu") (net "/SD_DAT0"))
 (via (at 4.345 34.7) (size 0.6) (drill 0.3) (layers "F.Cu" "B.Cu") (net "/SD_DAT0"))
 (segment (start 4.345 34.7) (end 14.2 34.7) (width 0.2) (layer "B.Cu") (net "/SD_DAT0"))
 (segment (start 14.2 34.7) (end 14.2 18.17) (width 0.2) (layer "B.Cu") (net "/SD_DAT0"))
 (segment (start 7.045 10.2365) (end 7.045 11.3865) (width 0.2) (layer "F.Cu") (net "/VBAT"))
 (via (at 7.045 11.3865) (size 0.6) (drill 0.3) (layers "F.Cu" "B.Cu") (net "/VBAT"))
 (segment (start 5.2 2.85) (end 8.5 2.85) (width 0.2) (layer "B.Cu") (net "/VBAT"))
 (segment (start 5.2 11.3865) (end 5.2 2.85) (width 0.2) (layer "B.Cu") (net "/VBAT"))
 (segment (start 7.045 11.3865) (end 5.2 11.3865) (width 0.2) (layer "B.Cu") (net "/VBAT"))
 (segment (start 7.045 8.3315) (end 8.945 6.9315) (width 0.2) (layer "F.Cu") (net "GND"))
 (segment (start 21.425 30.2) (end 21.425 31.9) (width 0.2) (layer "F.Cu") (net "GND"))
 (segment (start 9.95 22.9) (end 9.95 24.4) (width 0.2) (layer "F.Cu") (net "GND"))
 (segment (start 19.6 5.47) (end 17.9 5.47) (width 0.2) (layer "F.Cu") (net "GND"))
 (via (at 10.08 26.025) (size 0.6) (drill 0.3) (layers "F.Cu" "B.Cu") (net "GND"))
 (via (at 5.445 36.85) (size 0.6) (drill 0.3) (layers "F.Cu" "B.Cu") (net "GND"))
 (via (at 2.085 36.5) (size 0.6) (drill 0.3) (layers "F.Cu" "B.Cu") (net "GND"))
 (via (at 9.95 24.4) (size 0.6) (drill 0.3) (layers "F.Cu" "B.Cu") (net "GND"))
 (via (at 21.425 31.9) (size 0.6) (drill 0.3) (layers "F.Cu" "B.Cu") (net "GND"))
 (via (at 12.76 4.5215) (size 0.6) (drill 0.3) (layers "F.Cu" "B.Cu") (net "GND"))
 (via (at 8.945 6.9315) (size 0.6) (drill 0.3) (layers "F.Cu" "B.Cu") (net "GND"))
 (via (at 13.405 36.725) (size 0.6) (drill 0.3) (layers "F.Cu" "B.Cu") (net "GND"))
 (via (at 4.11 26.025) (size 0.6) (drill 0.3) (layers "F.Cu" "B.Cu") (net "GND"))
 (via (at 17.9 5.47) (size 0.6) (drill 0.3) (layers "F.Cu" "B.Cu") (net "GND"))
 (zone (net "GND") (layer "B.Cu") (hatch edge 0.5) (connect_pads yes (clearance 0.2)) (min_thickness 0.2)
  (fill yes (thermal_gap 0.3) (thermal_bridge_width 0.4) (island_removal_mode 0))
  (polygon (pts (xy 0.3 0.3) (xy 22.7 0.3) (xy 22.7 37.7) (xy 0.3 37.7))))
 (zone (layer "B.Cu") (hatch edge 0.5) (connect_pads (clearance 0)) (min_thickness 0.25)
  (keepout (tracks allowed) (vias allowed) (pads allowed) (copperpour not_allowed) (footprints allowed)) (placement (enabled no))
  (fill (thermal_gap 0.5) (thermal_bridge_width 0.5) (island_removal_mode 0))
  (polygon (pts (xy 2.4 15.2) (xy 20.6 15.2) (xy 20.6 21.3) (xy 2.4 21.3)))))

